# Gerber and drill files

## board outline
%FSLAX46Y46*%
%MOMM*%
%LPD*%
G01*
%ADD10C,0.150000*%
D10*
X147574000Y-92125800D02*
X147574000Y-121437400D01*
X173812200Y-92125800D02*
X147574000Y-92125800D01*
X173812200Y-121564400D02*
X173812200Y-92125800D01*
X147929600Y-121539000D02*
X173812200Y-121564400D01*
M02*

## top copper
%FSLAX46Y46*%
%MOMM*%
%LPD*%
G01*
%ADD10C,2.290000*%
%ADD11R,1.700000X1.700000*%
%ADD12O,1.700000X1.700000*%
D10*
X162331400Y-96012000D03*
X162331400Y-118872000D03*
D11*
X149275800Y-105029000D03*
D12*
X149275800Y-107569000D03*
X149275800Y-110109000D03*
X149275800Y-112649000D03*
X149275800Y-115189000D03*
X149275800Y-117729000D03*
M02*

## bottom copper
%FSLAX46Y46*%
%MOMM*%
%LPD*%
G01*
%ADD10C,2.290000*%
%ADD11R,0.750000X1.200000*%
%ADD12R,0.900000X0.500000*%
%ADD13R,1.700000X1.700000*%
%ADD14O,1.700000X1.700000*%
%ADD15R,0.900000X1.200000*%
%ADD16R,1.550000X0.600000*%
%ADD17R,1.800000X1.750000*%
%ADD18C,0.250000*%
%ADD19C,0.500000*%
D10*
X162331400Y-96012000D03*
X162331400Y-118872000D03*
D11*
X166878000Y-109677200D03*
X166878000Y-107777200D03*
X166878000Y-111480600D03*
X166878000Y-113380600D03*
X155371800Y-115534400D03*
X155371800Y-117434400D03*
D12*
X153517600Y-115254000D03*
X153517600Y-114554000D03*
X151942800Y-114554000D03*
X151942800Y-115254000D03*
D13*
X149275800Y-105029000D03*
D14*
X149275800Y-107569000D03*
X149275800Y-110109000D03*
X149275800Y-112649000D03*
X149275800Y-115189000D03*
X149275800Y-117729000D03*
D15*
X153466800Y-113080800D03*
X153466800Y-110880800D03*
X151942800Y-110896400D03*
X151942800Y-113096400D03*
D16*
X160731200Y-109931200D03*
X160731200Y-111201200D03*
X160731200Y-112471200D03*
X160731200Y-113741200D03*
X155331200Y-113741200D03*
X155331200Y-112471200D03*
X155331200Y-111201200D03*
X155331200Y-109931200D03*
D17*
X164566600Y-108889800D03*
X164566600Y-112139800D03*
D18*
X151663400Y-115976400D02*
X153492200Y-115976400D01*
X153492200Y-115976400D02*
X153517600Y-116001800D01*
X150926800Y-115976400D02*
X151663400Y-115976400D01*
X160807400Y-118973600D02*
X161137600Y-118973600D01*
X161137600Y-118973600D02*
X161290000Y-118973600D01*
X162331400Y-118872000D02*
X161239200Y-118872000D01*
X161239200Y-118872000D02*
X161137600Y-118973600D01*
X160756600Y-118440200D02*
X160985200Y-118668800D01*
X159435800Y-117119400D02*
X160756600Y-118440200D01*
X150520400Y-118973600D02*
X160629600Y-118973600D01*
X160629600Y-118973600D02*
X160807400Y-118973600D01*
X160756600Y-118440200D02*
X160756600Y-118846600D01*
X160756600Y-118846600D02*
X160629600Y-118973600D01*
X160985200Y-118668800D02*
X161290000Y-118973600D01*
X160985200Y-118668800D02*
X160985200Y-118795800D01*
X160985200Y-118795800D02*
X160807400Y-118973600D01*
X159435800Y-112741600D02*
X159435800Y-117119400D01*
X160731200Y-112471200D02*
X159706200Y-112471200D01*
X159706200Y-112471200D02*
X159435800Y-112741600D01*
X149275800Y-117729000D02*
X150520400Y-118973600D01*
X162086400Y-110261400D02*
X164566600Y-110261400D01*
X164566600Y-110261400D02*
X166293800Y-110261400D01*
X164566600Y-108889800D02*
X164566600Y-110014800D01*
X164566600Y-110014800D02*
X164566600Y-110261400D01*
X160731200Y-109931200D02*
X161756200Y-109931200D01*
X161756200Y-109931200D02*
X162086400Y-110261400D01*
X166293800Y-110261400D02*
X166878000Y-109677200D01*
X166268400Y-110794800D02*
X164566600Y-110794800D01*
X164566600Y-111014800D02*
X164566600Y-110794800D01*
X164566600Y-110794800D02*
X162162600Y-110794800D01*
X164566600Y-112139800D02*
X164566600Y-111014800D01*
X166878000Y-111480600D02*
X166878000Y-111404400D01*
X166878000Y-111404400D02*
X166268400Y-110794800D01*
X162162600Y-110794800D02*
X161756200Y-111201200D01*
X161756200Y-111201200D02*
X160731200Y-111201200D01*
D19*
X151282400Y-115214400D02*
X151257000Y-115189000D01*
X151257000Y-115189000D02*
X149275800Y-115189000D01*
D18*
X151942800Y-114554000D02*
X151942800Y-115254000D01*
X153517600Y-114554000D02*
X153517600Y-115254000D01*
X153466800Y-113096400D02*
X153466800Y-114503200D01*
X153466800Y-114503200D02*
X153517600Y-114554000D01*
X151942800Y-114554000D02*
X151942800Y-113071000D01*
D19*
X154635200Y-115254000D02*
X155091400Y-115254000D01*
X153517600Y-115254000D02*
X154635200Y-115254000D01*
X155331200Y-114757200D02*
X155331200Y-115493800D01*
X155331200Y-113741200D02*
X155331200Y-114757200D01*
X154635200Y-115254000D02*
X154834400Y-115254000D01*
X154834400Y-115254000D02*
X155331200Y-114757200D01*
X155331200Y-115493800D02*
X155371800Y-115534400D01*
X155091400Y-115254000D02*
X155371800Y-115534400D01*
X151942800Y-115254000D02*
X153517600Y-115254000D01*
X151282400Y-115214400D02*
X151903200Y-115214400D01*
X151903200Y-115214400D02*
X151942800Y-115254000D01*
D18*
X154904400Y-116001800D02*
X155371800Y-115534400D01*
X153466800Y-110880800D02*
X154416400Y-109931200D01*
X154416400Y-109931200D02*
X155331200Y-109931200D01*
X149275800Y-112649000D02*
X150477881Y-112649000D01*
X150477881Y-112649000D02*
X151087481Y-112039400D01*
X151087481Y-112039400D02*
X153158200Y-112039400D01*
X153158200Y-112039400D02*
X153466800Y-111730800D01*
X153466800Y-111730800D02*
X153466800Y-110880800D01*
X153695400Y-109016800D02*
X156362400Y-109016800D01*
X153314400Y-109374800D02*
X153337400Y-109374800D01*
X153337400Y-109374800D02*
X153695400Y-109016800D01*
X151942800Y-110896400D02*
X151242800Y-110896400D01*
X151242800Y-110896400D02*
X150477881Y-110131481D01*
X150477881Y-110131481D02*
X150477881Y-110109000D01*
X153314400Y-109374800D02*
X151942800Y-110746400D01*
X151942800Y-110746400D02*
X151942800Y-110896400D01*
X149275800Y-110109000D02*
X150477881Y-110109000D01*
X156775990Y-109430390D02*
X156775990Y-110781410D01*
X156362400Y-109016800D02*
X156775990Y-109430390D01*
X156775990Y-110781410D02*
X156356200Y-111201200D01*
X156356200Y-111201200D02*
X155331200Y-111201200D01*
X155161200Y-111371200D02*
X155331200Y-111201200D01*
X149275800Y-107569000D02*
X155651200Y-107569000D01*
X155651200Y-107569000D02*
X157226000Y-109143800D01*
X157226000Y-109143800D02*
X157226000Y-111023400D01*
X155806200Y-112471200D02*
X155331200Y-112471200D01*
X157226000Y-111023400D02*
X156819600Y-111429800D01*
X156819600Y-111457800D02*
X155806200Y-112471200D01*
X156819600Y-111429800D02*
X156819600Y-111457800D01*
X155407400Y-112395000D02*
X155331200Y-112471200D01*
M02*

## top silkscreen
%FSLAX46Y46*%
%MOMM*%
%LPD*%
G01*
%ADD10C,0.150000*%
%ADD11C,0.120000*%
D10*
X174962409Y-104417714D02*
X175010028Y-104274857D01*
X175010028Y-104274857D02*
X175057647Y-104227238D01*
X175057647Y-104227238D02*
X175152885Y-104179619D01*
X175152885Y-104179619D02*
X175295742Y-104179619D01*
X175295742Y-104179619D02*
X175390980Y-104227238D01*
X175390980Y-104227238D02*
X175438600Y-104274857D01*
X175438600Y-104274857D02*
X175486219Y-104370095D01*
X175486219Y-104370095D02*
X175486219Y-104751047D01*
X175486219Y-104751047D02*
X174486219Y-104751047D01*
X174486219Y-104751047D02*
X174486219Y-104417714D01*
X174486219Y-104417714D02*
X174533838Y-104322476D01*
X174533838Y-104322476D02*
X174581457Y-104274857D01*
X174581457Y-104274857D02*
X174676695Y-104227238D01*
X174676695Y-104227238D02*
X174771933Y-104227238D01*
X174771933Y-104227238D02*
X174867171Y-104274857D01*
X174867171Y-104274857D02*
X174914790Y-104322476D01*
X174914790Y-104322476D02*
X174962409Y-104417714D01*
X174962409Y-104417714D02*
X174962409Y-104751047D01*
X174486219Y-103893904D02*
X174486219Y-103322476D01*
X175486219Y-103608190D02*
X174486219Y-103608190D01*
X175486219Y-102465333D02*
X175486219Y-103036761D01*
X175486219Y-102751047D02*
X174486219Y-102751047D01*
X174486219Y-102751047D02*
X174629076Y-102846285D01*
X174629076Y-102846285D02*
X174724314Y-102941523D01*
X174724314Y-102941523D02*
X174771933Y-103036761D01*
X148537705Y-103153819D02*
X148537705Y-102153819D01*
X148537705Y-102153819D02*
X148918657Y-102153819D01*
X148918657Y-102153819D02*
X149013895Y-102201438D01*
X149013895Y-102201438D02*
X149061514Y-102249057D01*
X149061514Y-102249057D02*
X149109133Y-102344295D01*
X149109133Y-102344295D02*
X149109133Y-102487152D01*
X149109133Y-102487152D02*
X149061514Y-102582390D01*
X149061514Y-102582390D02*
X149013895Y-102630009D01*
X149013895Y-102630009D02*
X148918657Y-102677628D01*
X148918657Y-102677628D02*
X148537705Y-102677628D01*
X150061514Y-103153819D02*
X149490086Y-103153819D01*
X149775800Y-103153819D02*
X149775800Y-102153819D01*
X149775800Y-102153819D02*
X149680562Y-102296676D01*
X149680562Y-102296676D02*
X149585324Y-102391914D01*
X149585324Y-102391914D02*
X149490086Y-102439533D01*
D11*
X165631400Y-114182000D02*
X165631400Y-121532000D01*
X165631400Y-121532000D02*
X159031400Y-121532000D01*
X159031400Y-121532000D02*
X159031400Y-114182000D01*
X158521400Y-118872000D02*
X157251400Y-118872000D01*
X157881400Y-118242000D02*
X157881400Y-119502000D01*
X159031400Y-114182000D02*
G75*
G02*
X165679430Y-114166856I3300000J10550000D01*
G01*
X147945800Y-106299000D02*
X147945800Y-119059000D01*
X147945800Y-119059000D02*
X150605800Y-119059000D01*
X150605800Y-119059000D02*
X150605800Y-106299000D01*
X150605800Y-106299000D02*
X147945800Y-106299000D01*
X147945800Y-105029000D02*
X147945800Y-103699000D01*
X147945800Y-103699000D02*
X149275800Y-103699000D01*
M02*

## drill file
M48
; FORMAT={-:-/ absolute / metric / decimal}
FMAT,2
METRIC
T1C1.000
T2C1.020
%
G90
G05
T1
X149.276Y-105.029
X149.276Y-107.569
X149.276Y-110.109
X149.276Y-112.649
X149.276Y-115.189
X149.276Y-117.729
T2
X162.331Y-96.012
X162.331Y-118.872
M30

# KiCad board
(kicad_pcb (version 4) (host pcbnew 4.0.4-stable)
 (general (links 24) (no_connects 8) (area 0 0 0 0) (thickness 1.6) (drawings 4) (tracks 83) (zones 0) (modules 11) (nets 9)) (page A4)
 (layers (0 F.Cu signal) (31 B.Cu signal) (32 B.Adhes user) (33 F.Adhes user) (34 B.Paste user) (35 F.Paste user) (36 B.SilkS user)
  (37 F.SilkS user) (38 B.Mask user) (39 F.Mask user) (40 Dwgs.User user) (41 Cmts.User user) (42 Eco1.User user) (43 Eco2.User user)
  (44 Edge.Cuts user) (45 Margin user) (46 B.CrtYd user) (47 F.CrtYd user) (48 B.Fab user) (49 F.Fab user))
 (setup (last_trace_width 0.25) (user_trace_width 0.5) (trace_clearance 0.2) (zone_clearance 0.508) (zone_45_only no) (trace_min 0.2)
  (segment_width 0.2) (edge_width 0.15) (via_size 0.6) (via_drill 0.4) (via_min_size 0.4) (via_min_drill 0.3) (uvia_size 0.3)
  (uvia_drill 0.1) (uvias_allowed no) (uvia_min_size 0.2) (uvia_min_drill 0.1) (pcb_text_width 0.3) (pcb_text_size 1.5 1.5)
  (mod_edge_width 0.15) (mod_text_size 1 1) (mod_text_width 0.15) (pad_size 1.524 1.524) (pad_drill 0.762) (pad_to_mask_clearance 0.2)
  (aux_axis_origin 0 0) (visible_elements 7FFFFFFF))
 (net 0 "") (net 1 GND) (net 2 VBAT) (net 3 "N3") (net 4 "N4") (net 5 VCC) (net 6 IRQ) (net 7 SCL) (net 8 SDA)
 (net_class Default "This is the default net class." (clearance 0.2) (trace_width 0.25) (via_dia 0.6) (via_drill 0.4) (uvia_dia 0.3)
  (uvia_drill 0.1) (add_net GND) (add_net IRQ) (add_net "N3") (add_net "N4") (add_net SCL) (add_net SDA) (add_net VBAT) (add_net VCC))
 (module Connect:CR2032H (layer F.Cu) (at 162.3314 118.872 270)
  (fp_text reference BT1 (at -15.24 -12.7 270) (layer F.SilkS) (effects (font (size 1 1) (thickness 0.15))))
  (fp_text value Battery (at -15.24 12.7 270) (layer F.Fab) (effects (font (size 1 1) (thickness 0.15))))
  (fp_line (start -4.69 -3.3) (end 2.66 -3.3) (layer F.SilkS) (width 0.12))
  (fp_line (start 2.66 -3.3) (end 2.66 3.3) (layer F.SilkS) (width 0.12))
  (fp_line (start 2.66 3.3) (end -4.69 3.3) (layer F.SilkS) (width 0.12))
  (fp_line (start 0 3.81) (end 0 5.08) (layer F.SilkS) (width 0.12))
  (fp_line (start -0.63 4.45) (end 0.63 4.45) (layer F.SilkS) (width 0.12))
  (fp_arc (start -15.24 0) (end -4.69 3.3) (angle 325) (layer F.SilkS) (width 0.12))
  (pad 2 thru_hole circle (at -22.86 0 270) (size 2.29 2.29) (drill 1.02) (layers *.Cu *.Mask) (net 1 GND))
  (pad 1 thru_hole circle (at 0 0 270) (size 2.29 2.29) (drill 1.02) (layers *.Cu *.Mask) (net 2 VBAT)))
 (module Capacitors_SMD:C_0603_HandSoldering (layer B.Cu) (at 166.878 108.7272 90)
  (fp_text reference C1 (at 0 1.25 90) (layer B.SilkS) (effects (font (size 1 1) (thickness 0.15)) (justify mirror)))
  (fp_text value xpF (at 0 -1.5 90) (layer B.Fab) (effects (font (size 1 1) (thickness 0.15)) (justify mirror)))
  (pad 1 smd rect (at -0.95 0 90) (size 1.2 0.75) (layers B.Cu B.Paste B.Mask) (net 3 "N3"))
  (pad 2 smd rect (at 0.95 0 90) (size 1.2 0.75) (layers B.Cu B.Paste B.Mask) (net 1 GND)))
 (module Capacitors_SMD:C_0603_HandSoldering (layer B.Cu) (at 166.878 112.4306 270)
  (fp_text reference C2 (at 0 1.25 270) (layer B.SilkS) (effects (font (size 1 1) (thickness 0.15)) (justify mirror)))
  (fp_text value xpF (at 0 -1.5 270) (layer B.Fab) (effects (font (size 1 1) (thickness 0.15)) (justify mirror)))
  (pad 1 smd rect (at -0.95 0 270) (size 1.2 0.75) (layers B.Cu B.Paste B.Mask) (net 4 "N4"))
  (pad 2 smd rect (at 0.95 0 270) (size 1.2 0.75) (layers B.Cu B.Paste B.Mask) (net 1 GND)))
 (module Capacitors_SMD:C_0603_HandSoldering (layer B.Cu) (at 155.3718 116.4844 270)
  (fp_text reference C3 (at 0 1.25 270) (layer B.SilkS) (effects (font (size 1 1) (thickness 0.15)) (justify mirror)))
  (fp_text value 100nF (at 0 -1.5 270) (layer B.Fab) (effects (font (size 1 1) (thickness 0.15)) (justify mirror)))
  (pad 1 smd rect (at -0.95 0 270) (size 1.2 0.75) (layers B.Cu B.Paste B.Mask) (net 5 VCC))
  (pad 2 smd rect (at 0.95 0 270) (size 1.2 0.75) (layers B.Cu B.Paste B.Mask) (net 1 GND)))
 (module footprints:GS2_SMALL (layer B.Cu) (at 153.5176 114.554)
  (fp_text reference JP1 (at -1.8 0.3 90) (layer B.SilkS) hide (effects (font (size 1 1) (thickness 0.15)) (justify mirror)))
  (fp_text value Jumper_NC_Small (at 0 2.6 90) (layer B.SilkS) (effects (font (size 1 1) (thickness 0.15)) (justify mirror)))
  (pad 1 smd rect (at 0 0.7) (size 0.9 0.5) (layers B.Cu B.Paste B.Mask) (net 5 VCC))
  (pad 2 smd rect (at 0 0) (size 0.9 0.5) (layers B.Cu B.Paste B.Mask) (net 5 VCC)))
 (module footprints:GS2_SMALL (layer B.Cu) (at 151.9428 115.254 180)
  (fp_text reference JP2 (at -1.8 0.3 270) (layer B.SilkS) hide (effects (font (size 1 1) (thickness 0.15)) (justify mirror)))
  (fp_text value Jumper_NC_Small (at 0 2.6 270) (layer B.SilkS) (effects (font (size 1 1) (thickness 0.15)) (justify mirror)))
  (pad 1 smd rect (at 0 0.7 180) (size 0.9 0.5) (layers B.Cu B.Paste B.Mask) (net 5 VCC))
  (pad 2 smd rect (at 0 0 180) (size 0.9 0.5) (layers B.Cu B.Paste B.Mask) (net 5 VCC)))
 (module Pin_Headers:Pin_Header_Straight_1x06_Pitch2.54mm (layer F.Cu) (at 149.2758 105.029)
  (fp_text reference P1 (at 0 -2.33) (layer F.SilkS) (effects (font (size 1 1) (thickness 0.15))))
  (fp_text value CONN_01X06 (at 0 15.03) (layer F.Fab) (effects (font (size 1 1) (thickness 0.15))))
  (fp_line (start -1.33 1.27) (end -1.33 14.03) (layer F.SilkS) (width 0.12))
  (fp_line (start -1.33 14.03) (end 1.33 14.03) (layer F.SilkS) (width 0.12))
  (fp_line (start 1.33 14.03) (end 1.33 1.27) (layer F.SilkS) (width 0.12))
  (fp_line (start 1.33 1.27) (end -1.33 1.27) (layer F.SilkS) (width 0.12))
  (fp_line (start -1.33 0) (end -1.33 -1.33) (layer F.SilkS) (width 0.12))
  (fp_line (start -1.33 -1.33) (end 0 -1.33) (layer F.SilkS) (width 0.12))
  (pad 1 thru_hole rect (at 0 0) (size 1.7 1.7) (drill 1) (layers *.Cu *.Mask) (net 1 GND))
  (pad 2 thru_hole oval (at 0 2.54) (size 1.7 1.7) (drill 1) (layers *.Cu *.Mask) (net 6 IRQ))
  (pad 3 thru_hole oval (at 0 5.08) (size 1.7 1.7) (drill 1) (layers *.Cu *.Mask) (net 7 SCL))
  (pad 4 thru_hole oval (at 0 7.62) (size 1.7 1.7) (drill 1) (layers *.Cu *.Mask) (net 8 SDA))
  (pad 5 thru_hole oval (at 0 10.16) (size 1.7 1.7) (drill 1) (layers *.Cu *.Mask) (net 5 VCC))
  (pad 6 thru_hole oval (at 0 12.7) (size 1.7 1.7) (drill 1) (layers *.Cu *.Mask) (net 2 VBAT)))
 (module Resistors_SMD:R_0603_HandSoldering (layer B.Cu) (at 153.4668 111.9808 90)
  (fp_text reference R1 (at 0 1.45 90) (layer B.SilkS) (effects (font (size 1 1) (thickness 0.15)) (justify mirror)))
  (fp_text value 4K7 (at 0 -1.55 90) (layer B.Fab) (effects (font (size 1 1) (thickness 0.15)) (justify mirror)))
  (pad 1 smd rect (at -1.1 0 90) (size 1.2 0.9) (layers B.Cu B.Paste B.Mask) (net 5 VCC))
  (pad 2 smd rect (at 1.1 0 90) (size 1.2 0.9) (layers B.Cu B.Paste B.Mask) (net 8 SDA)))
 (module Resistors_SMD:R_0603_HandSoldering (layer B.Cu) (at 151.9428 111.9964 270)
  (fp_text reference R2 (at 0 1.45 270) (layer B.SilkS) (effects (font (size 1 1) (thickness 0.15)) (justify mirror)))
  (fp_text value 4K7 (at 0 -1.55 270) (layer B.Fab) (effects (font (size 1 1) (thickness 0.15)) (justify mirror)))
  (pad 1 smd rect (at -1.1 0 270) (size 1.2 0.9) (layers B.Cu B.Paste B.Mask) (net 7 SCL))
  (pad 2 smd rect (at 1.1 0 270) (size 1.2 0.9) (layers B.Cu B.Paste B.Mask) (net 5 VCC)))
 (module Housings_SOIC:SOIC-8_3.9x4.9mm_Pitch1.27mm (layer B.Cu) (at 158.0312 111.8362 180)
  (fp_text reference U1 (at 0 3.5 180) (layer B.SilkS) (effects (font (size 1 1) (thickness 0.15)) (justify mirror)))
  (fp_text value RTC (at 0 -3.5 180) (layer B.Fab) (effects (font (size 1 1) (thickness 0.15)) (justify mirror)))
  (pad 1 smd rect (at -2.7 1.905 180) (size 1.55 0.6) (layers B.Cu B.Paste B.Mask) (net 3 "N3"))
  (pad 2 smd rect (at -2.7 0.635 180) (size 1.55 0.6) (layers B.Cu B.Paste B.Mask) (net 4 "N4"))
  (pad 3 smd rect (at -2.7 -0.635 180) (size 1.55 0.6) (layers B.Cu B.Paste B.Mask) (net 2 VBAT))
  (pad 4 smd rect (at -2.7 -1.905 180) (size 1.55 0.6) (layers B.Cu B.Paste B.Mask) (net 1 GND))
  (pad 5 smd rect (at 2.7 -1.905 180) (size 1.55 0.6) (layers B.Cu B.Paste B.Mask) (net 5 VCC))
  (pad 6 smd rect (at 2.7 -0.635 180) (size 1.55 0.6) (layers B.Cu B.Paste B.Mask) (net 6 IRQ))
  (pad 7 smd rect (at 2.7 0.635 180) (size 1.55 0.6) (layers B.Cu B.Paste B.Mask) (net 7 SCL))
  (pad 8 smd rect (at 2.7 1.905 180) (size 1.55 0.6) (layers B.Cu B.Paste B.Mask) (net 8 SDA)))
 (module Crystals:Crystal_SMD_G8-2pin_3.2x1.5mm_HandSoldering (layer B.Cu) (at 164.5666 110.5148 270)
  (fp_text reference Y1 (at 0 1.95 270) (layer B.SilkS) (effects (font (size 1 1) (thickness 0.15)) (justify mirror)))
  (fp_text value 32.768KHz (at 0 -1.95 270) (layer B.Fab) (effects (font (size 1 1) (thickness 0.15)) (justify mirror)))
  (pad 1 smd rect (at -1.625 0 270) (size 1.75 1.8) (layers B.Cu B.Paste B.Mask) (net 3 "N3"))
  (pad 2 smd rect (at 1.625 0 270) (size 1.75 1.8) (layers B.Cu B.Paste B.Mask) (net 4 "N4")))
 (gr_line (start 147.574 92.1258) (end 147.574 121.4374) (layer Edge.Cuts) (width 0.15))
 (gr_line (start 173.8122 92.1258) (end 147.574 92.1258) (layer Edge.Cuts) (width 0.15))
 (gr_line (start 173.8122 121.5644) (end 173.8122 92.1258) (layer Edge.Cuts) (width 0.15))
 (gr_line (start 147.9296 121.539) (end 173.8122 121.5644) (layer Edge.Cuts) (width 0.15))
 (segment (start 151.6634 115.9764) (end 153.4922 115.9764) (width 0.25) (layer B.Cu) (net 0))
 (segment (start 153.4922 115.9764) (end 153.5176 116.0018) (width 0.25) (layer B.Cu) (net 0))
 (segment (start 150.9268 115.9764) (end 151.6634 115.9764) (width 0.25) (layer B.Cu) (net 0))
 (segment (start 160.8074 118.9736) (end 161.1376 118.9736) (width 0.25) (layer B.Cu) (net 2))
 (segment (start 161.1376 118.9736) (end 161.29 118.9736) (width 0.25) (layer B.Cu) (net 2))
 (segment (start 162.3314 118.872) (end 161.2392 118.872) (width 0.25) (layer B.Cu) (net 2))
 (segment (start 161.2392 118.872) (end 161.1376 118.9736) (width 0.25) (layer B.Cu) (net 2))
 (segment (start 160.7566 118.4402) (end 160.9852 118.6688) (width 0.25) (layer B.Cu) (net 2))
 (segment (start 159.4358 117.1194) (end 160.7566 118.4402) (width 0.25) (layer B.Cu) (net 2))
 (segment (start 150.5204 118.9736) (end 160.6296 118.9736) (width 0.25) (layer B.Cu) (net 2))
 (segment (start 160.6296 118.9736) (end 160.8074 118.9736) (width 0.25) (layer B.Cu) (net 2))
 (segment (start 160.7566 118.4402) (end 160.7566 118.8466) (width 0.25) (layer B.Cu) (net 2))
 (segment (start 160.7566 118.8466) (end 160.6296 118.9736) (width 0.25) (layer B.Cu) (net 2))
 (segment (start 160.9852 118.6688) (end 161.29 118.9736) (width 0.25) (layer B.Cu) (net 2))
 (segment (start 160.9852 118.6688) (end 160.9852 118.7958) (width 0.25) (layer B.Cu) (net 2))
 (segment (start 160.9852 118.7958) (end 160.8074 118.9736) (width 0.25) (layer B.Cu) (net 2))
 (segment (start 159.4358 112.7416) (end 159.4358 117.1194) (width 0.25) (layer B.Cu) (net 2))
 (segment (start 160.7312 112.4712) (end 159.7062 112.4712) (width 0.25) (layer B.Cu) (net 2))
 (segment (start 159.7062 112.4712) (end 159.4358 112.7416) (width 0.25) (layer B.Cu) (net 2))
 (segment (start 149.2758 117.729) (end 150.5204 118.9736) (width 0.25) (layer B.Cu) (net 2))
 (segment (start 162.0864 110.2614) (end 164.5666 110.2614) (width 0.25) (layer B.Cu) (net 3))
 (segment (start 164.5666 110.2614) (end 166.2938 110.2614) (width 0.25) (layer B.Cu) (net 3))
 (segment (start 164.5666 108.8898) (end 164.5666 110.0148) (width 0.25) (layer B.Cu) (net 3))
 (segment (start 164.5666 110.0148) (end 164.5666 110.2614) (width 0.25) (layer B.Cu) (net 3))
 (segment (start 160.7312 109.9312) (end 161.7562 109.9312) (width 0.25) (layer B.Cu) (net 3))
 (segment (start 161.7562 109.9312) (end 162.0864 110.2614) (width 0.25) (layer B.Cu) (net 3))
 (segment (start 166.2938 110.2614) (end 166.878 109.6772) (width 0.25) (layer B.Cu) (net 3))
 (segment (start 166.2684 110.7948) (end 164.5666 110.7948) (width 0.25) (layer B.Cu) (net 4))
 (segment (start 164.5666 111.0148) (end 164.5666 110.7948) (width 0.25) (layer B.Cu) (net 4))
 (segment (start 164.5666 110.7948) (end 162.1626 110.7948) (width 0.25) (layer B.Cu) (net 4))
 (segment (start 164.5666 112.1398) (end 164.5666 111.0148) (width 0.25) (layer B.Cu) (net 4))
 (segment (start 166.878 111.4806) (end 166.878 111.4044) (width 0.25) (layer B.Cu) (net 4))
 (segment (start 166.878 111.4044) (end 166.2684 110.7948) (width 0.25) (layer B.Cu) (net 4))
 (segment (start 162.1626 110.7948) (end 161.7562 111.2012) (width 0.25) (layer B.Cu) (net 4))
 (segment (start 161.7562 111.2012) (end 160.7312 111.2012) (width 0.25) (layer B.Cu) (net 4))
 (segment (start 151.2824 115.2144) (end 151.257 115.189) (width 0.5) (layer B.Cu) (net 5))
 (segment (start 151.257 115.189) (end 149.2758 115.189) (width 0.5) (layer B.Cu) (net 5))
 (segment (start 151.9428 114.554) (end 151.9428 115.254) (width 0.25) (layer B.Cu) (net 5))
 (segment (start 153.5176 114.554) (end 153.5176 115.254) (width 0.25) (layer B.Cu) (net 5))
 (segment (start 153.4668 113.0964) (end 153.4668 114.5032) (width 0.25) (layer B.Cu) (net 5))
 (segment (start 153.4668 114.5032) (end 153.5176 114.554) (width 0.25) (layer B.Cu) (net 5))
 (segment (start 151.9428 114.554) (end 151.9428 113.071) (width 0.25) (layer B.Cu) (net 5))
 (segment (start 154.6352 115.254) (end 155.0914 115.254) (width 0.5) (layer B.Cu) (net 5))
 (segment (start 153.5176 115.254) (end 154.6352 115.254) (width 0.5) (layer B.Cu) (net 5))
 (segment (start 155.3312 114.7572) (end 155.3312 115.4938) (width 0.5) (layer B.Cu) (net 5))
 (segment (start 155.3312 113.7412) (end 155.3312 114.7572) (width 0.5) (layer B.Cu) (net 5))
 (segment (start 154.6352 115.254) (end 154.8344 115.254) (width 0.5) (layer B.Cu) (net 5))
 (segment (start 154.8344 115.254) (end 155.3312 114.7572) (width 0.5) (layer B.Cu) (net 5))
 (segment (start 155.3312 115.4938) (end 155.3718 115.5344) (width 0.5) (layer B.Cu) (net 5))
 (segment (start 155.0914 115.254) (end 155.3718 115.5344) (width 0.5) (layer B.Cu) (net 5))
 (segment (start 151.9428 115.254) (end 153.5176 115.254) (width 0.5) (layer B.Cu) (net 5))
 (segment (start 151.2824 115.2144) (end 151.9032 115.2144) (width 0.5) (layer B.Cu) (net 5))
 (segment (start 151.9032 115.2144) (end 151.9428 115.254) (width 0.5) (layer B.Cu) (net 5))
 (segment (start 154.9044 116.0018) (end 155.3718 115.5344) (width 0.25) (layer B.Cu) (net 5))
 (segment (start 153.4668 110.8808) (end 154.4164 109.9312) (width 0.25) (layer B.Cu) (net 8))
 (segment (start 154.4164 109.9312) (end 155.3312 109.9312) (width 0.25) (layer B.Cu) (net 8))
 (segment (start 149.2758 112.649) (end 150.477881 112.649) (width 0.25) (layer B.Cu) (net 8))
 (segment (start 150.477881 112.649) (end 151.087481 112.0394) (width 0.25) (layer B.Cu) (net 8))
 (segment (start 151.087481 112.0394) (end 153.1582 112.0394) (width 0.25) (layer B.Cu) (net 8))
 (segment (start 153.1582 112.0394) (end 153.4668 111.7308) (width 0.25) (layer B.Cu) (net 8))
 (segment (start 153.4668 111.7308) (end 153.4668 110.8808) (width 0.25) (layer B.Cu) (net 8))
 (segment (start 153.6954 109.0168) (end 156.3624 109.0168) (width 0.25) (layer B.Cu) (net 7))
 (segment (start 153.3144 109.3748) (end 153.3374 109.3748) (width 0.25) (layer B.Cu) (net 7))
 (segment (start 153.3374 109.3748) (end 153.6954 109.0168) (width 0.25) (layer B.Cu) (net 7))
 (segment (start 151.9428 110.8964) (end 151.2428 110.8964) (width 0.25) (layer B.Cu) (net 7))
 (segment (start 151.2428 110.8964) (end 150.477881 110.131481) (width 0.25) (layer B.Cu) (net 7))
 (segment (start 150.477881 110.131481) (end 150.477881 110.109) (width 0.25) (layer B.Cu) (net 7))
 (segment (start 153.3144 109.3748) (end 151.9428 110.7464) (width 0.25) (layer B.Cu) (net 7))
 (segment (start 151.9428 110.7464) (end 151.9428 110.8964) (width 0.25) (layer B.Cu) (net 7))
 (segment (start 149.2758 110.109) (end 150.477881 110.109) (width 0.25) (layer B.Cu) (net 7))
 (segment (start 156.77599 109.43039) (end 156.77599 110.78141) (width 0.25) (layer B.Cu) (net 7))
 (segment (start 156.3624 109.0168) (end 156.77599 109.43039) (width 0.25) (layer B.Cu) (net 7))
 (segment (start 156.77599 110.78141) (end 156.3562 111.2012) (width 0.25) (layer B.Cu) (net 7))
 (segment (start 156.3562 111.2012) (end 155.3312 111.2012) (width 0.25) (layer B.Cu) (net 7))
 (segment (start 155.1612 111.3712) (end 155.3312 111.2012) (width 0.25) (layer B.Cu) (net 7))
 (segment (start 149.2758 107.569) (end 155.6512 107.569) (width 0.25) (layer B.Cu) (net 6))
 (segment (start 155.6512 107.569) (end 157.226 109.1438) (width 0.25) (layer B.Cu) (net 6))
 (segment (start 157.226 109.1438) (end 157.226 111.0234) (width 0.25) (layer B.Cu) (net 6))
 (segment (start 155.8062 112.4712) (end 155.3312 112.4712) (width 0.25) (layer B.Cu) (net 6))
 (segment (start 157.226 111.0234) (end 156.8196 111.4298) (width 0.25) (layer B.Cu) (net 6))
 (segment (start 156.8196 111.4578) (end 155.8062 112.4712) (width 0.25) (layer B.Cu) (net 6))
 (segment (start 156.8196 111.4298) (end 156.8196 111.4578) (width 0.25) (layer B.Cu) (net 6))
 (segment (start 155.4074 112.395) (end 155.3312 112.4712) (width 0.25) (layer B.Cu) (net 6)))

